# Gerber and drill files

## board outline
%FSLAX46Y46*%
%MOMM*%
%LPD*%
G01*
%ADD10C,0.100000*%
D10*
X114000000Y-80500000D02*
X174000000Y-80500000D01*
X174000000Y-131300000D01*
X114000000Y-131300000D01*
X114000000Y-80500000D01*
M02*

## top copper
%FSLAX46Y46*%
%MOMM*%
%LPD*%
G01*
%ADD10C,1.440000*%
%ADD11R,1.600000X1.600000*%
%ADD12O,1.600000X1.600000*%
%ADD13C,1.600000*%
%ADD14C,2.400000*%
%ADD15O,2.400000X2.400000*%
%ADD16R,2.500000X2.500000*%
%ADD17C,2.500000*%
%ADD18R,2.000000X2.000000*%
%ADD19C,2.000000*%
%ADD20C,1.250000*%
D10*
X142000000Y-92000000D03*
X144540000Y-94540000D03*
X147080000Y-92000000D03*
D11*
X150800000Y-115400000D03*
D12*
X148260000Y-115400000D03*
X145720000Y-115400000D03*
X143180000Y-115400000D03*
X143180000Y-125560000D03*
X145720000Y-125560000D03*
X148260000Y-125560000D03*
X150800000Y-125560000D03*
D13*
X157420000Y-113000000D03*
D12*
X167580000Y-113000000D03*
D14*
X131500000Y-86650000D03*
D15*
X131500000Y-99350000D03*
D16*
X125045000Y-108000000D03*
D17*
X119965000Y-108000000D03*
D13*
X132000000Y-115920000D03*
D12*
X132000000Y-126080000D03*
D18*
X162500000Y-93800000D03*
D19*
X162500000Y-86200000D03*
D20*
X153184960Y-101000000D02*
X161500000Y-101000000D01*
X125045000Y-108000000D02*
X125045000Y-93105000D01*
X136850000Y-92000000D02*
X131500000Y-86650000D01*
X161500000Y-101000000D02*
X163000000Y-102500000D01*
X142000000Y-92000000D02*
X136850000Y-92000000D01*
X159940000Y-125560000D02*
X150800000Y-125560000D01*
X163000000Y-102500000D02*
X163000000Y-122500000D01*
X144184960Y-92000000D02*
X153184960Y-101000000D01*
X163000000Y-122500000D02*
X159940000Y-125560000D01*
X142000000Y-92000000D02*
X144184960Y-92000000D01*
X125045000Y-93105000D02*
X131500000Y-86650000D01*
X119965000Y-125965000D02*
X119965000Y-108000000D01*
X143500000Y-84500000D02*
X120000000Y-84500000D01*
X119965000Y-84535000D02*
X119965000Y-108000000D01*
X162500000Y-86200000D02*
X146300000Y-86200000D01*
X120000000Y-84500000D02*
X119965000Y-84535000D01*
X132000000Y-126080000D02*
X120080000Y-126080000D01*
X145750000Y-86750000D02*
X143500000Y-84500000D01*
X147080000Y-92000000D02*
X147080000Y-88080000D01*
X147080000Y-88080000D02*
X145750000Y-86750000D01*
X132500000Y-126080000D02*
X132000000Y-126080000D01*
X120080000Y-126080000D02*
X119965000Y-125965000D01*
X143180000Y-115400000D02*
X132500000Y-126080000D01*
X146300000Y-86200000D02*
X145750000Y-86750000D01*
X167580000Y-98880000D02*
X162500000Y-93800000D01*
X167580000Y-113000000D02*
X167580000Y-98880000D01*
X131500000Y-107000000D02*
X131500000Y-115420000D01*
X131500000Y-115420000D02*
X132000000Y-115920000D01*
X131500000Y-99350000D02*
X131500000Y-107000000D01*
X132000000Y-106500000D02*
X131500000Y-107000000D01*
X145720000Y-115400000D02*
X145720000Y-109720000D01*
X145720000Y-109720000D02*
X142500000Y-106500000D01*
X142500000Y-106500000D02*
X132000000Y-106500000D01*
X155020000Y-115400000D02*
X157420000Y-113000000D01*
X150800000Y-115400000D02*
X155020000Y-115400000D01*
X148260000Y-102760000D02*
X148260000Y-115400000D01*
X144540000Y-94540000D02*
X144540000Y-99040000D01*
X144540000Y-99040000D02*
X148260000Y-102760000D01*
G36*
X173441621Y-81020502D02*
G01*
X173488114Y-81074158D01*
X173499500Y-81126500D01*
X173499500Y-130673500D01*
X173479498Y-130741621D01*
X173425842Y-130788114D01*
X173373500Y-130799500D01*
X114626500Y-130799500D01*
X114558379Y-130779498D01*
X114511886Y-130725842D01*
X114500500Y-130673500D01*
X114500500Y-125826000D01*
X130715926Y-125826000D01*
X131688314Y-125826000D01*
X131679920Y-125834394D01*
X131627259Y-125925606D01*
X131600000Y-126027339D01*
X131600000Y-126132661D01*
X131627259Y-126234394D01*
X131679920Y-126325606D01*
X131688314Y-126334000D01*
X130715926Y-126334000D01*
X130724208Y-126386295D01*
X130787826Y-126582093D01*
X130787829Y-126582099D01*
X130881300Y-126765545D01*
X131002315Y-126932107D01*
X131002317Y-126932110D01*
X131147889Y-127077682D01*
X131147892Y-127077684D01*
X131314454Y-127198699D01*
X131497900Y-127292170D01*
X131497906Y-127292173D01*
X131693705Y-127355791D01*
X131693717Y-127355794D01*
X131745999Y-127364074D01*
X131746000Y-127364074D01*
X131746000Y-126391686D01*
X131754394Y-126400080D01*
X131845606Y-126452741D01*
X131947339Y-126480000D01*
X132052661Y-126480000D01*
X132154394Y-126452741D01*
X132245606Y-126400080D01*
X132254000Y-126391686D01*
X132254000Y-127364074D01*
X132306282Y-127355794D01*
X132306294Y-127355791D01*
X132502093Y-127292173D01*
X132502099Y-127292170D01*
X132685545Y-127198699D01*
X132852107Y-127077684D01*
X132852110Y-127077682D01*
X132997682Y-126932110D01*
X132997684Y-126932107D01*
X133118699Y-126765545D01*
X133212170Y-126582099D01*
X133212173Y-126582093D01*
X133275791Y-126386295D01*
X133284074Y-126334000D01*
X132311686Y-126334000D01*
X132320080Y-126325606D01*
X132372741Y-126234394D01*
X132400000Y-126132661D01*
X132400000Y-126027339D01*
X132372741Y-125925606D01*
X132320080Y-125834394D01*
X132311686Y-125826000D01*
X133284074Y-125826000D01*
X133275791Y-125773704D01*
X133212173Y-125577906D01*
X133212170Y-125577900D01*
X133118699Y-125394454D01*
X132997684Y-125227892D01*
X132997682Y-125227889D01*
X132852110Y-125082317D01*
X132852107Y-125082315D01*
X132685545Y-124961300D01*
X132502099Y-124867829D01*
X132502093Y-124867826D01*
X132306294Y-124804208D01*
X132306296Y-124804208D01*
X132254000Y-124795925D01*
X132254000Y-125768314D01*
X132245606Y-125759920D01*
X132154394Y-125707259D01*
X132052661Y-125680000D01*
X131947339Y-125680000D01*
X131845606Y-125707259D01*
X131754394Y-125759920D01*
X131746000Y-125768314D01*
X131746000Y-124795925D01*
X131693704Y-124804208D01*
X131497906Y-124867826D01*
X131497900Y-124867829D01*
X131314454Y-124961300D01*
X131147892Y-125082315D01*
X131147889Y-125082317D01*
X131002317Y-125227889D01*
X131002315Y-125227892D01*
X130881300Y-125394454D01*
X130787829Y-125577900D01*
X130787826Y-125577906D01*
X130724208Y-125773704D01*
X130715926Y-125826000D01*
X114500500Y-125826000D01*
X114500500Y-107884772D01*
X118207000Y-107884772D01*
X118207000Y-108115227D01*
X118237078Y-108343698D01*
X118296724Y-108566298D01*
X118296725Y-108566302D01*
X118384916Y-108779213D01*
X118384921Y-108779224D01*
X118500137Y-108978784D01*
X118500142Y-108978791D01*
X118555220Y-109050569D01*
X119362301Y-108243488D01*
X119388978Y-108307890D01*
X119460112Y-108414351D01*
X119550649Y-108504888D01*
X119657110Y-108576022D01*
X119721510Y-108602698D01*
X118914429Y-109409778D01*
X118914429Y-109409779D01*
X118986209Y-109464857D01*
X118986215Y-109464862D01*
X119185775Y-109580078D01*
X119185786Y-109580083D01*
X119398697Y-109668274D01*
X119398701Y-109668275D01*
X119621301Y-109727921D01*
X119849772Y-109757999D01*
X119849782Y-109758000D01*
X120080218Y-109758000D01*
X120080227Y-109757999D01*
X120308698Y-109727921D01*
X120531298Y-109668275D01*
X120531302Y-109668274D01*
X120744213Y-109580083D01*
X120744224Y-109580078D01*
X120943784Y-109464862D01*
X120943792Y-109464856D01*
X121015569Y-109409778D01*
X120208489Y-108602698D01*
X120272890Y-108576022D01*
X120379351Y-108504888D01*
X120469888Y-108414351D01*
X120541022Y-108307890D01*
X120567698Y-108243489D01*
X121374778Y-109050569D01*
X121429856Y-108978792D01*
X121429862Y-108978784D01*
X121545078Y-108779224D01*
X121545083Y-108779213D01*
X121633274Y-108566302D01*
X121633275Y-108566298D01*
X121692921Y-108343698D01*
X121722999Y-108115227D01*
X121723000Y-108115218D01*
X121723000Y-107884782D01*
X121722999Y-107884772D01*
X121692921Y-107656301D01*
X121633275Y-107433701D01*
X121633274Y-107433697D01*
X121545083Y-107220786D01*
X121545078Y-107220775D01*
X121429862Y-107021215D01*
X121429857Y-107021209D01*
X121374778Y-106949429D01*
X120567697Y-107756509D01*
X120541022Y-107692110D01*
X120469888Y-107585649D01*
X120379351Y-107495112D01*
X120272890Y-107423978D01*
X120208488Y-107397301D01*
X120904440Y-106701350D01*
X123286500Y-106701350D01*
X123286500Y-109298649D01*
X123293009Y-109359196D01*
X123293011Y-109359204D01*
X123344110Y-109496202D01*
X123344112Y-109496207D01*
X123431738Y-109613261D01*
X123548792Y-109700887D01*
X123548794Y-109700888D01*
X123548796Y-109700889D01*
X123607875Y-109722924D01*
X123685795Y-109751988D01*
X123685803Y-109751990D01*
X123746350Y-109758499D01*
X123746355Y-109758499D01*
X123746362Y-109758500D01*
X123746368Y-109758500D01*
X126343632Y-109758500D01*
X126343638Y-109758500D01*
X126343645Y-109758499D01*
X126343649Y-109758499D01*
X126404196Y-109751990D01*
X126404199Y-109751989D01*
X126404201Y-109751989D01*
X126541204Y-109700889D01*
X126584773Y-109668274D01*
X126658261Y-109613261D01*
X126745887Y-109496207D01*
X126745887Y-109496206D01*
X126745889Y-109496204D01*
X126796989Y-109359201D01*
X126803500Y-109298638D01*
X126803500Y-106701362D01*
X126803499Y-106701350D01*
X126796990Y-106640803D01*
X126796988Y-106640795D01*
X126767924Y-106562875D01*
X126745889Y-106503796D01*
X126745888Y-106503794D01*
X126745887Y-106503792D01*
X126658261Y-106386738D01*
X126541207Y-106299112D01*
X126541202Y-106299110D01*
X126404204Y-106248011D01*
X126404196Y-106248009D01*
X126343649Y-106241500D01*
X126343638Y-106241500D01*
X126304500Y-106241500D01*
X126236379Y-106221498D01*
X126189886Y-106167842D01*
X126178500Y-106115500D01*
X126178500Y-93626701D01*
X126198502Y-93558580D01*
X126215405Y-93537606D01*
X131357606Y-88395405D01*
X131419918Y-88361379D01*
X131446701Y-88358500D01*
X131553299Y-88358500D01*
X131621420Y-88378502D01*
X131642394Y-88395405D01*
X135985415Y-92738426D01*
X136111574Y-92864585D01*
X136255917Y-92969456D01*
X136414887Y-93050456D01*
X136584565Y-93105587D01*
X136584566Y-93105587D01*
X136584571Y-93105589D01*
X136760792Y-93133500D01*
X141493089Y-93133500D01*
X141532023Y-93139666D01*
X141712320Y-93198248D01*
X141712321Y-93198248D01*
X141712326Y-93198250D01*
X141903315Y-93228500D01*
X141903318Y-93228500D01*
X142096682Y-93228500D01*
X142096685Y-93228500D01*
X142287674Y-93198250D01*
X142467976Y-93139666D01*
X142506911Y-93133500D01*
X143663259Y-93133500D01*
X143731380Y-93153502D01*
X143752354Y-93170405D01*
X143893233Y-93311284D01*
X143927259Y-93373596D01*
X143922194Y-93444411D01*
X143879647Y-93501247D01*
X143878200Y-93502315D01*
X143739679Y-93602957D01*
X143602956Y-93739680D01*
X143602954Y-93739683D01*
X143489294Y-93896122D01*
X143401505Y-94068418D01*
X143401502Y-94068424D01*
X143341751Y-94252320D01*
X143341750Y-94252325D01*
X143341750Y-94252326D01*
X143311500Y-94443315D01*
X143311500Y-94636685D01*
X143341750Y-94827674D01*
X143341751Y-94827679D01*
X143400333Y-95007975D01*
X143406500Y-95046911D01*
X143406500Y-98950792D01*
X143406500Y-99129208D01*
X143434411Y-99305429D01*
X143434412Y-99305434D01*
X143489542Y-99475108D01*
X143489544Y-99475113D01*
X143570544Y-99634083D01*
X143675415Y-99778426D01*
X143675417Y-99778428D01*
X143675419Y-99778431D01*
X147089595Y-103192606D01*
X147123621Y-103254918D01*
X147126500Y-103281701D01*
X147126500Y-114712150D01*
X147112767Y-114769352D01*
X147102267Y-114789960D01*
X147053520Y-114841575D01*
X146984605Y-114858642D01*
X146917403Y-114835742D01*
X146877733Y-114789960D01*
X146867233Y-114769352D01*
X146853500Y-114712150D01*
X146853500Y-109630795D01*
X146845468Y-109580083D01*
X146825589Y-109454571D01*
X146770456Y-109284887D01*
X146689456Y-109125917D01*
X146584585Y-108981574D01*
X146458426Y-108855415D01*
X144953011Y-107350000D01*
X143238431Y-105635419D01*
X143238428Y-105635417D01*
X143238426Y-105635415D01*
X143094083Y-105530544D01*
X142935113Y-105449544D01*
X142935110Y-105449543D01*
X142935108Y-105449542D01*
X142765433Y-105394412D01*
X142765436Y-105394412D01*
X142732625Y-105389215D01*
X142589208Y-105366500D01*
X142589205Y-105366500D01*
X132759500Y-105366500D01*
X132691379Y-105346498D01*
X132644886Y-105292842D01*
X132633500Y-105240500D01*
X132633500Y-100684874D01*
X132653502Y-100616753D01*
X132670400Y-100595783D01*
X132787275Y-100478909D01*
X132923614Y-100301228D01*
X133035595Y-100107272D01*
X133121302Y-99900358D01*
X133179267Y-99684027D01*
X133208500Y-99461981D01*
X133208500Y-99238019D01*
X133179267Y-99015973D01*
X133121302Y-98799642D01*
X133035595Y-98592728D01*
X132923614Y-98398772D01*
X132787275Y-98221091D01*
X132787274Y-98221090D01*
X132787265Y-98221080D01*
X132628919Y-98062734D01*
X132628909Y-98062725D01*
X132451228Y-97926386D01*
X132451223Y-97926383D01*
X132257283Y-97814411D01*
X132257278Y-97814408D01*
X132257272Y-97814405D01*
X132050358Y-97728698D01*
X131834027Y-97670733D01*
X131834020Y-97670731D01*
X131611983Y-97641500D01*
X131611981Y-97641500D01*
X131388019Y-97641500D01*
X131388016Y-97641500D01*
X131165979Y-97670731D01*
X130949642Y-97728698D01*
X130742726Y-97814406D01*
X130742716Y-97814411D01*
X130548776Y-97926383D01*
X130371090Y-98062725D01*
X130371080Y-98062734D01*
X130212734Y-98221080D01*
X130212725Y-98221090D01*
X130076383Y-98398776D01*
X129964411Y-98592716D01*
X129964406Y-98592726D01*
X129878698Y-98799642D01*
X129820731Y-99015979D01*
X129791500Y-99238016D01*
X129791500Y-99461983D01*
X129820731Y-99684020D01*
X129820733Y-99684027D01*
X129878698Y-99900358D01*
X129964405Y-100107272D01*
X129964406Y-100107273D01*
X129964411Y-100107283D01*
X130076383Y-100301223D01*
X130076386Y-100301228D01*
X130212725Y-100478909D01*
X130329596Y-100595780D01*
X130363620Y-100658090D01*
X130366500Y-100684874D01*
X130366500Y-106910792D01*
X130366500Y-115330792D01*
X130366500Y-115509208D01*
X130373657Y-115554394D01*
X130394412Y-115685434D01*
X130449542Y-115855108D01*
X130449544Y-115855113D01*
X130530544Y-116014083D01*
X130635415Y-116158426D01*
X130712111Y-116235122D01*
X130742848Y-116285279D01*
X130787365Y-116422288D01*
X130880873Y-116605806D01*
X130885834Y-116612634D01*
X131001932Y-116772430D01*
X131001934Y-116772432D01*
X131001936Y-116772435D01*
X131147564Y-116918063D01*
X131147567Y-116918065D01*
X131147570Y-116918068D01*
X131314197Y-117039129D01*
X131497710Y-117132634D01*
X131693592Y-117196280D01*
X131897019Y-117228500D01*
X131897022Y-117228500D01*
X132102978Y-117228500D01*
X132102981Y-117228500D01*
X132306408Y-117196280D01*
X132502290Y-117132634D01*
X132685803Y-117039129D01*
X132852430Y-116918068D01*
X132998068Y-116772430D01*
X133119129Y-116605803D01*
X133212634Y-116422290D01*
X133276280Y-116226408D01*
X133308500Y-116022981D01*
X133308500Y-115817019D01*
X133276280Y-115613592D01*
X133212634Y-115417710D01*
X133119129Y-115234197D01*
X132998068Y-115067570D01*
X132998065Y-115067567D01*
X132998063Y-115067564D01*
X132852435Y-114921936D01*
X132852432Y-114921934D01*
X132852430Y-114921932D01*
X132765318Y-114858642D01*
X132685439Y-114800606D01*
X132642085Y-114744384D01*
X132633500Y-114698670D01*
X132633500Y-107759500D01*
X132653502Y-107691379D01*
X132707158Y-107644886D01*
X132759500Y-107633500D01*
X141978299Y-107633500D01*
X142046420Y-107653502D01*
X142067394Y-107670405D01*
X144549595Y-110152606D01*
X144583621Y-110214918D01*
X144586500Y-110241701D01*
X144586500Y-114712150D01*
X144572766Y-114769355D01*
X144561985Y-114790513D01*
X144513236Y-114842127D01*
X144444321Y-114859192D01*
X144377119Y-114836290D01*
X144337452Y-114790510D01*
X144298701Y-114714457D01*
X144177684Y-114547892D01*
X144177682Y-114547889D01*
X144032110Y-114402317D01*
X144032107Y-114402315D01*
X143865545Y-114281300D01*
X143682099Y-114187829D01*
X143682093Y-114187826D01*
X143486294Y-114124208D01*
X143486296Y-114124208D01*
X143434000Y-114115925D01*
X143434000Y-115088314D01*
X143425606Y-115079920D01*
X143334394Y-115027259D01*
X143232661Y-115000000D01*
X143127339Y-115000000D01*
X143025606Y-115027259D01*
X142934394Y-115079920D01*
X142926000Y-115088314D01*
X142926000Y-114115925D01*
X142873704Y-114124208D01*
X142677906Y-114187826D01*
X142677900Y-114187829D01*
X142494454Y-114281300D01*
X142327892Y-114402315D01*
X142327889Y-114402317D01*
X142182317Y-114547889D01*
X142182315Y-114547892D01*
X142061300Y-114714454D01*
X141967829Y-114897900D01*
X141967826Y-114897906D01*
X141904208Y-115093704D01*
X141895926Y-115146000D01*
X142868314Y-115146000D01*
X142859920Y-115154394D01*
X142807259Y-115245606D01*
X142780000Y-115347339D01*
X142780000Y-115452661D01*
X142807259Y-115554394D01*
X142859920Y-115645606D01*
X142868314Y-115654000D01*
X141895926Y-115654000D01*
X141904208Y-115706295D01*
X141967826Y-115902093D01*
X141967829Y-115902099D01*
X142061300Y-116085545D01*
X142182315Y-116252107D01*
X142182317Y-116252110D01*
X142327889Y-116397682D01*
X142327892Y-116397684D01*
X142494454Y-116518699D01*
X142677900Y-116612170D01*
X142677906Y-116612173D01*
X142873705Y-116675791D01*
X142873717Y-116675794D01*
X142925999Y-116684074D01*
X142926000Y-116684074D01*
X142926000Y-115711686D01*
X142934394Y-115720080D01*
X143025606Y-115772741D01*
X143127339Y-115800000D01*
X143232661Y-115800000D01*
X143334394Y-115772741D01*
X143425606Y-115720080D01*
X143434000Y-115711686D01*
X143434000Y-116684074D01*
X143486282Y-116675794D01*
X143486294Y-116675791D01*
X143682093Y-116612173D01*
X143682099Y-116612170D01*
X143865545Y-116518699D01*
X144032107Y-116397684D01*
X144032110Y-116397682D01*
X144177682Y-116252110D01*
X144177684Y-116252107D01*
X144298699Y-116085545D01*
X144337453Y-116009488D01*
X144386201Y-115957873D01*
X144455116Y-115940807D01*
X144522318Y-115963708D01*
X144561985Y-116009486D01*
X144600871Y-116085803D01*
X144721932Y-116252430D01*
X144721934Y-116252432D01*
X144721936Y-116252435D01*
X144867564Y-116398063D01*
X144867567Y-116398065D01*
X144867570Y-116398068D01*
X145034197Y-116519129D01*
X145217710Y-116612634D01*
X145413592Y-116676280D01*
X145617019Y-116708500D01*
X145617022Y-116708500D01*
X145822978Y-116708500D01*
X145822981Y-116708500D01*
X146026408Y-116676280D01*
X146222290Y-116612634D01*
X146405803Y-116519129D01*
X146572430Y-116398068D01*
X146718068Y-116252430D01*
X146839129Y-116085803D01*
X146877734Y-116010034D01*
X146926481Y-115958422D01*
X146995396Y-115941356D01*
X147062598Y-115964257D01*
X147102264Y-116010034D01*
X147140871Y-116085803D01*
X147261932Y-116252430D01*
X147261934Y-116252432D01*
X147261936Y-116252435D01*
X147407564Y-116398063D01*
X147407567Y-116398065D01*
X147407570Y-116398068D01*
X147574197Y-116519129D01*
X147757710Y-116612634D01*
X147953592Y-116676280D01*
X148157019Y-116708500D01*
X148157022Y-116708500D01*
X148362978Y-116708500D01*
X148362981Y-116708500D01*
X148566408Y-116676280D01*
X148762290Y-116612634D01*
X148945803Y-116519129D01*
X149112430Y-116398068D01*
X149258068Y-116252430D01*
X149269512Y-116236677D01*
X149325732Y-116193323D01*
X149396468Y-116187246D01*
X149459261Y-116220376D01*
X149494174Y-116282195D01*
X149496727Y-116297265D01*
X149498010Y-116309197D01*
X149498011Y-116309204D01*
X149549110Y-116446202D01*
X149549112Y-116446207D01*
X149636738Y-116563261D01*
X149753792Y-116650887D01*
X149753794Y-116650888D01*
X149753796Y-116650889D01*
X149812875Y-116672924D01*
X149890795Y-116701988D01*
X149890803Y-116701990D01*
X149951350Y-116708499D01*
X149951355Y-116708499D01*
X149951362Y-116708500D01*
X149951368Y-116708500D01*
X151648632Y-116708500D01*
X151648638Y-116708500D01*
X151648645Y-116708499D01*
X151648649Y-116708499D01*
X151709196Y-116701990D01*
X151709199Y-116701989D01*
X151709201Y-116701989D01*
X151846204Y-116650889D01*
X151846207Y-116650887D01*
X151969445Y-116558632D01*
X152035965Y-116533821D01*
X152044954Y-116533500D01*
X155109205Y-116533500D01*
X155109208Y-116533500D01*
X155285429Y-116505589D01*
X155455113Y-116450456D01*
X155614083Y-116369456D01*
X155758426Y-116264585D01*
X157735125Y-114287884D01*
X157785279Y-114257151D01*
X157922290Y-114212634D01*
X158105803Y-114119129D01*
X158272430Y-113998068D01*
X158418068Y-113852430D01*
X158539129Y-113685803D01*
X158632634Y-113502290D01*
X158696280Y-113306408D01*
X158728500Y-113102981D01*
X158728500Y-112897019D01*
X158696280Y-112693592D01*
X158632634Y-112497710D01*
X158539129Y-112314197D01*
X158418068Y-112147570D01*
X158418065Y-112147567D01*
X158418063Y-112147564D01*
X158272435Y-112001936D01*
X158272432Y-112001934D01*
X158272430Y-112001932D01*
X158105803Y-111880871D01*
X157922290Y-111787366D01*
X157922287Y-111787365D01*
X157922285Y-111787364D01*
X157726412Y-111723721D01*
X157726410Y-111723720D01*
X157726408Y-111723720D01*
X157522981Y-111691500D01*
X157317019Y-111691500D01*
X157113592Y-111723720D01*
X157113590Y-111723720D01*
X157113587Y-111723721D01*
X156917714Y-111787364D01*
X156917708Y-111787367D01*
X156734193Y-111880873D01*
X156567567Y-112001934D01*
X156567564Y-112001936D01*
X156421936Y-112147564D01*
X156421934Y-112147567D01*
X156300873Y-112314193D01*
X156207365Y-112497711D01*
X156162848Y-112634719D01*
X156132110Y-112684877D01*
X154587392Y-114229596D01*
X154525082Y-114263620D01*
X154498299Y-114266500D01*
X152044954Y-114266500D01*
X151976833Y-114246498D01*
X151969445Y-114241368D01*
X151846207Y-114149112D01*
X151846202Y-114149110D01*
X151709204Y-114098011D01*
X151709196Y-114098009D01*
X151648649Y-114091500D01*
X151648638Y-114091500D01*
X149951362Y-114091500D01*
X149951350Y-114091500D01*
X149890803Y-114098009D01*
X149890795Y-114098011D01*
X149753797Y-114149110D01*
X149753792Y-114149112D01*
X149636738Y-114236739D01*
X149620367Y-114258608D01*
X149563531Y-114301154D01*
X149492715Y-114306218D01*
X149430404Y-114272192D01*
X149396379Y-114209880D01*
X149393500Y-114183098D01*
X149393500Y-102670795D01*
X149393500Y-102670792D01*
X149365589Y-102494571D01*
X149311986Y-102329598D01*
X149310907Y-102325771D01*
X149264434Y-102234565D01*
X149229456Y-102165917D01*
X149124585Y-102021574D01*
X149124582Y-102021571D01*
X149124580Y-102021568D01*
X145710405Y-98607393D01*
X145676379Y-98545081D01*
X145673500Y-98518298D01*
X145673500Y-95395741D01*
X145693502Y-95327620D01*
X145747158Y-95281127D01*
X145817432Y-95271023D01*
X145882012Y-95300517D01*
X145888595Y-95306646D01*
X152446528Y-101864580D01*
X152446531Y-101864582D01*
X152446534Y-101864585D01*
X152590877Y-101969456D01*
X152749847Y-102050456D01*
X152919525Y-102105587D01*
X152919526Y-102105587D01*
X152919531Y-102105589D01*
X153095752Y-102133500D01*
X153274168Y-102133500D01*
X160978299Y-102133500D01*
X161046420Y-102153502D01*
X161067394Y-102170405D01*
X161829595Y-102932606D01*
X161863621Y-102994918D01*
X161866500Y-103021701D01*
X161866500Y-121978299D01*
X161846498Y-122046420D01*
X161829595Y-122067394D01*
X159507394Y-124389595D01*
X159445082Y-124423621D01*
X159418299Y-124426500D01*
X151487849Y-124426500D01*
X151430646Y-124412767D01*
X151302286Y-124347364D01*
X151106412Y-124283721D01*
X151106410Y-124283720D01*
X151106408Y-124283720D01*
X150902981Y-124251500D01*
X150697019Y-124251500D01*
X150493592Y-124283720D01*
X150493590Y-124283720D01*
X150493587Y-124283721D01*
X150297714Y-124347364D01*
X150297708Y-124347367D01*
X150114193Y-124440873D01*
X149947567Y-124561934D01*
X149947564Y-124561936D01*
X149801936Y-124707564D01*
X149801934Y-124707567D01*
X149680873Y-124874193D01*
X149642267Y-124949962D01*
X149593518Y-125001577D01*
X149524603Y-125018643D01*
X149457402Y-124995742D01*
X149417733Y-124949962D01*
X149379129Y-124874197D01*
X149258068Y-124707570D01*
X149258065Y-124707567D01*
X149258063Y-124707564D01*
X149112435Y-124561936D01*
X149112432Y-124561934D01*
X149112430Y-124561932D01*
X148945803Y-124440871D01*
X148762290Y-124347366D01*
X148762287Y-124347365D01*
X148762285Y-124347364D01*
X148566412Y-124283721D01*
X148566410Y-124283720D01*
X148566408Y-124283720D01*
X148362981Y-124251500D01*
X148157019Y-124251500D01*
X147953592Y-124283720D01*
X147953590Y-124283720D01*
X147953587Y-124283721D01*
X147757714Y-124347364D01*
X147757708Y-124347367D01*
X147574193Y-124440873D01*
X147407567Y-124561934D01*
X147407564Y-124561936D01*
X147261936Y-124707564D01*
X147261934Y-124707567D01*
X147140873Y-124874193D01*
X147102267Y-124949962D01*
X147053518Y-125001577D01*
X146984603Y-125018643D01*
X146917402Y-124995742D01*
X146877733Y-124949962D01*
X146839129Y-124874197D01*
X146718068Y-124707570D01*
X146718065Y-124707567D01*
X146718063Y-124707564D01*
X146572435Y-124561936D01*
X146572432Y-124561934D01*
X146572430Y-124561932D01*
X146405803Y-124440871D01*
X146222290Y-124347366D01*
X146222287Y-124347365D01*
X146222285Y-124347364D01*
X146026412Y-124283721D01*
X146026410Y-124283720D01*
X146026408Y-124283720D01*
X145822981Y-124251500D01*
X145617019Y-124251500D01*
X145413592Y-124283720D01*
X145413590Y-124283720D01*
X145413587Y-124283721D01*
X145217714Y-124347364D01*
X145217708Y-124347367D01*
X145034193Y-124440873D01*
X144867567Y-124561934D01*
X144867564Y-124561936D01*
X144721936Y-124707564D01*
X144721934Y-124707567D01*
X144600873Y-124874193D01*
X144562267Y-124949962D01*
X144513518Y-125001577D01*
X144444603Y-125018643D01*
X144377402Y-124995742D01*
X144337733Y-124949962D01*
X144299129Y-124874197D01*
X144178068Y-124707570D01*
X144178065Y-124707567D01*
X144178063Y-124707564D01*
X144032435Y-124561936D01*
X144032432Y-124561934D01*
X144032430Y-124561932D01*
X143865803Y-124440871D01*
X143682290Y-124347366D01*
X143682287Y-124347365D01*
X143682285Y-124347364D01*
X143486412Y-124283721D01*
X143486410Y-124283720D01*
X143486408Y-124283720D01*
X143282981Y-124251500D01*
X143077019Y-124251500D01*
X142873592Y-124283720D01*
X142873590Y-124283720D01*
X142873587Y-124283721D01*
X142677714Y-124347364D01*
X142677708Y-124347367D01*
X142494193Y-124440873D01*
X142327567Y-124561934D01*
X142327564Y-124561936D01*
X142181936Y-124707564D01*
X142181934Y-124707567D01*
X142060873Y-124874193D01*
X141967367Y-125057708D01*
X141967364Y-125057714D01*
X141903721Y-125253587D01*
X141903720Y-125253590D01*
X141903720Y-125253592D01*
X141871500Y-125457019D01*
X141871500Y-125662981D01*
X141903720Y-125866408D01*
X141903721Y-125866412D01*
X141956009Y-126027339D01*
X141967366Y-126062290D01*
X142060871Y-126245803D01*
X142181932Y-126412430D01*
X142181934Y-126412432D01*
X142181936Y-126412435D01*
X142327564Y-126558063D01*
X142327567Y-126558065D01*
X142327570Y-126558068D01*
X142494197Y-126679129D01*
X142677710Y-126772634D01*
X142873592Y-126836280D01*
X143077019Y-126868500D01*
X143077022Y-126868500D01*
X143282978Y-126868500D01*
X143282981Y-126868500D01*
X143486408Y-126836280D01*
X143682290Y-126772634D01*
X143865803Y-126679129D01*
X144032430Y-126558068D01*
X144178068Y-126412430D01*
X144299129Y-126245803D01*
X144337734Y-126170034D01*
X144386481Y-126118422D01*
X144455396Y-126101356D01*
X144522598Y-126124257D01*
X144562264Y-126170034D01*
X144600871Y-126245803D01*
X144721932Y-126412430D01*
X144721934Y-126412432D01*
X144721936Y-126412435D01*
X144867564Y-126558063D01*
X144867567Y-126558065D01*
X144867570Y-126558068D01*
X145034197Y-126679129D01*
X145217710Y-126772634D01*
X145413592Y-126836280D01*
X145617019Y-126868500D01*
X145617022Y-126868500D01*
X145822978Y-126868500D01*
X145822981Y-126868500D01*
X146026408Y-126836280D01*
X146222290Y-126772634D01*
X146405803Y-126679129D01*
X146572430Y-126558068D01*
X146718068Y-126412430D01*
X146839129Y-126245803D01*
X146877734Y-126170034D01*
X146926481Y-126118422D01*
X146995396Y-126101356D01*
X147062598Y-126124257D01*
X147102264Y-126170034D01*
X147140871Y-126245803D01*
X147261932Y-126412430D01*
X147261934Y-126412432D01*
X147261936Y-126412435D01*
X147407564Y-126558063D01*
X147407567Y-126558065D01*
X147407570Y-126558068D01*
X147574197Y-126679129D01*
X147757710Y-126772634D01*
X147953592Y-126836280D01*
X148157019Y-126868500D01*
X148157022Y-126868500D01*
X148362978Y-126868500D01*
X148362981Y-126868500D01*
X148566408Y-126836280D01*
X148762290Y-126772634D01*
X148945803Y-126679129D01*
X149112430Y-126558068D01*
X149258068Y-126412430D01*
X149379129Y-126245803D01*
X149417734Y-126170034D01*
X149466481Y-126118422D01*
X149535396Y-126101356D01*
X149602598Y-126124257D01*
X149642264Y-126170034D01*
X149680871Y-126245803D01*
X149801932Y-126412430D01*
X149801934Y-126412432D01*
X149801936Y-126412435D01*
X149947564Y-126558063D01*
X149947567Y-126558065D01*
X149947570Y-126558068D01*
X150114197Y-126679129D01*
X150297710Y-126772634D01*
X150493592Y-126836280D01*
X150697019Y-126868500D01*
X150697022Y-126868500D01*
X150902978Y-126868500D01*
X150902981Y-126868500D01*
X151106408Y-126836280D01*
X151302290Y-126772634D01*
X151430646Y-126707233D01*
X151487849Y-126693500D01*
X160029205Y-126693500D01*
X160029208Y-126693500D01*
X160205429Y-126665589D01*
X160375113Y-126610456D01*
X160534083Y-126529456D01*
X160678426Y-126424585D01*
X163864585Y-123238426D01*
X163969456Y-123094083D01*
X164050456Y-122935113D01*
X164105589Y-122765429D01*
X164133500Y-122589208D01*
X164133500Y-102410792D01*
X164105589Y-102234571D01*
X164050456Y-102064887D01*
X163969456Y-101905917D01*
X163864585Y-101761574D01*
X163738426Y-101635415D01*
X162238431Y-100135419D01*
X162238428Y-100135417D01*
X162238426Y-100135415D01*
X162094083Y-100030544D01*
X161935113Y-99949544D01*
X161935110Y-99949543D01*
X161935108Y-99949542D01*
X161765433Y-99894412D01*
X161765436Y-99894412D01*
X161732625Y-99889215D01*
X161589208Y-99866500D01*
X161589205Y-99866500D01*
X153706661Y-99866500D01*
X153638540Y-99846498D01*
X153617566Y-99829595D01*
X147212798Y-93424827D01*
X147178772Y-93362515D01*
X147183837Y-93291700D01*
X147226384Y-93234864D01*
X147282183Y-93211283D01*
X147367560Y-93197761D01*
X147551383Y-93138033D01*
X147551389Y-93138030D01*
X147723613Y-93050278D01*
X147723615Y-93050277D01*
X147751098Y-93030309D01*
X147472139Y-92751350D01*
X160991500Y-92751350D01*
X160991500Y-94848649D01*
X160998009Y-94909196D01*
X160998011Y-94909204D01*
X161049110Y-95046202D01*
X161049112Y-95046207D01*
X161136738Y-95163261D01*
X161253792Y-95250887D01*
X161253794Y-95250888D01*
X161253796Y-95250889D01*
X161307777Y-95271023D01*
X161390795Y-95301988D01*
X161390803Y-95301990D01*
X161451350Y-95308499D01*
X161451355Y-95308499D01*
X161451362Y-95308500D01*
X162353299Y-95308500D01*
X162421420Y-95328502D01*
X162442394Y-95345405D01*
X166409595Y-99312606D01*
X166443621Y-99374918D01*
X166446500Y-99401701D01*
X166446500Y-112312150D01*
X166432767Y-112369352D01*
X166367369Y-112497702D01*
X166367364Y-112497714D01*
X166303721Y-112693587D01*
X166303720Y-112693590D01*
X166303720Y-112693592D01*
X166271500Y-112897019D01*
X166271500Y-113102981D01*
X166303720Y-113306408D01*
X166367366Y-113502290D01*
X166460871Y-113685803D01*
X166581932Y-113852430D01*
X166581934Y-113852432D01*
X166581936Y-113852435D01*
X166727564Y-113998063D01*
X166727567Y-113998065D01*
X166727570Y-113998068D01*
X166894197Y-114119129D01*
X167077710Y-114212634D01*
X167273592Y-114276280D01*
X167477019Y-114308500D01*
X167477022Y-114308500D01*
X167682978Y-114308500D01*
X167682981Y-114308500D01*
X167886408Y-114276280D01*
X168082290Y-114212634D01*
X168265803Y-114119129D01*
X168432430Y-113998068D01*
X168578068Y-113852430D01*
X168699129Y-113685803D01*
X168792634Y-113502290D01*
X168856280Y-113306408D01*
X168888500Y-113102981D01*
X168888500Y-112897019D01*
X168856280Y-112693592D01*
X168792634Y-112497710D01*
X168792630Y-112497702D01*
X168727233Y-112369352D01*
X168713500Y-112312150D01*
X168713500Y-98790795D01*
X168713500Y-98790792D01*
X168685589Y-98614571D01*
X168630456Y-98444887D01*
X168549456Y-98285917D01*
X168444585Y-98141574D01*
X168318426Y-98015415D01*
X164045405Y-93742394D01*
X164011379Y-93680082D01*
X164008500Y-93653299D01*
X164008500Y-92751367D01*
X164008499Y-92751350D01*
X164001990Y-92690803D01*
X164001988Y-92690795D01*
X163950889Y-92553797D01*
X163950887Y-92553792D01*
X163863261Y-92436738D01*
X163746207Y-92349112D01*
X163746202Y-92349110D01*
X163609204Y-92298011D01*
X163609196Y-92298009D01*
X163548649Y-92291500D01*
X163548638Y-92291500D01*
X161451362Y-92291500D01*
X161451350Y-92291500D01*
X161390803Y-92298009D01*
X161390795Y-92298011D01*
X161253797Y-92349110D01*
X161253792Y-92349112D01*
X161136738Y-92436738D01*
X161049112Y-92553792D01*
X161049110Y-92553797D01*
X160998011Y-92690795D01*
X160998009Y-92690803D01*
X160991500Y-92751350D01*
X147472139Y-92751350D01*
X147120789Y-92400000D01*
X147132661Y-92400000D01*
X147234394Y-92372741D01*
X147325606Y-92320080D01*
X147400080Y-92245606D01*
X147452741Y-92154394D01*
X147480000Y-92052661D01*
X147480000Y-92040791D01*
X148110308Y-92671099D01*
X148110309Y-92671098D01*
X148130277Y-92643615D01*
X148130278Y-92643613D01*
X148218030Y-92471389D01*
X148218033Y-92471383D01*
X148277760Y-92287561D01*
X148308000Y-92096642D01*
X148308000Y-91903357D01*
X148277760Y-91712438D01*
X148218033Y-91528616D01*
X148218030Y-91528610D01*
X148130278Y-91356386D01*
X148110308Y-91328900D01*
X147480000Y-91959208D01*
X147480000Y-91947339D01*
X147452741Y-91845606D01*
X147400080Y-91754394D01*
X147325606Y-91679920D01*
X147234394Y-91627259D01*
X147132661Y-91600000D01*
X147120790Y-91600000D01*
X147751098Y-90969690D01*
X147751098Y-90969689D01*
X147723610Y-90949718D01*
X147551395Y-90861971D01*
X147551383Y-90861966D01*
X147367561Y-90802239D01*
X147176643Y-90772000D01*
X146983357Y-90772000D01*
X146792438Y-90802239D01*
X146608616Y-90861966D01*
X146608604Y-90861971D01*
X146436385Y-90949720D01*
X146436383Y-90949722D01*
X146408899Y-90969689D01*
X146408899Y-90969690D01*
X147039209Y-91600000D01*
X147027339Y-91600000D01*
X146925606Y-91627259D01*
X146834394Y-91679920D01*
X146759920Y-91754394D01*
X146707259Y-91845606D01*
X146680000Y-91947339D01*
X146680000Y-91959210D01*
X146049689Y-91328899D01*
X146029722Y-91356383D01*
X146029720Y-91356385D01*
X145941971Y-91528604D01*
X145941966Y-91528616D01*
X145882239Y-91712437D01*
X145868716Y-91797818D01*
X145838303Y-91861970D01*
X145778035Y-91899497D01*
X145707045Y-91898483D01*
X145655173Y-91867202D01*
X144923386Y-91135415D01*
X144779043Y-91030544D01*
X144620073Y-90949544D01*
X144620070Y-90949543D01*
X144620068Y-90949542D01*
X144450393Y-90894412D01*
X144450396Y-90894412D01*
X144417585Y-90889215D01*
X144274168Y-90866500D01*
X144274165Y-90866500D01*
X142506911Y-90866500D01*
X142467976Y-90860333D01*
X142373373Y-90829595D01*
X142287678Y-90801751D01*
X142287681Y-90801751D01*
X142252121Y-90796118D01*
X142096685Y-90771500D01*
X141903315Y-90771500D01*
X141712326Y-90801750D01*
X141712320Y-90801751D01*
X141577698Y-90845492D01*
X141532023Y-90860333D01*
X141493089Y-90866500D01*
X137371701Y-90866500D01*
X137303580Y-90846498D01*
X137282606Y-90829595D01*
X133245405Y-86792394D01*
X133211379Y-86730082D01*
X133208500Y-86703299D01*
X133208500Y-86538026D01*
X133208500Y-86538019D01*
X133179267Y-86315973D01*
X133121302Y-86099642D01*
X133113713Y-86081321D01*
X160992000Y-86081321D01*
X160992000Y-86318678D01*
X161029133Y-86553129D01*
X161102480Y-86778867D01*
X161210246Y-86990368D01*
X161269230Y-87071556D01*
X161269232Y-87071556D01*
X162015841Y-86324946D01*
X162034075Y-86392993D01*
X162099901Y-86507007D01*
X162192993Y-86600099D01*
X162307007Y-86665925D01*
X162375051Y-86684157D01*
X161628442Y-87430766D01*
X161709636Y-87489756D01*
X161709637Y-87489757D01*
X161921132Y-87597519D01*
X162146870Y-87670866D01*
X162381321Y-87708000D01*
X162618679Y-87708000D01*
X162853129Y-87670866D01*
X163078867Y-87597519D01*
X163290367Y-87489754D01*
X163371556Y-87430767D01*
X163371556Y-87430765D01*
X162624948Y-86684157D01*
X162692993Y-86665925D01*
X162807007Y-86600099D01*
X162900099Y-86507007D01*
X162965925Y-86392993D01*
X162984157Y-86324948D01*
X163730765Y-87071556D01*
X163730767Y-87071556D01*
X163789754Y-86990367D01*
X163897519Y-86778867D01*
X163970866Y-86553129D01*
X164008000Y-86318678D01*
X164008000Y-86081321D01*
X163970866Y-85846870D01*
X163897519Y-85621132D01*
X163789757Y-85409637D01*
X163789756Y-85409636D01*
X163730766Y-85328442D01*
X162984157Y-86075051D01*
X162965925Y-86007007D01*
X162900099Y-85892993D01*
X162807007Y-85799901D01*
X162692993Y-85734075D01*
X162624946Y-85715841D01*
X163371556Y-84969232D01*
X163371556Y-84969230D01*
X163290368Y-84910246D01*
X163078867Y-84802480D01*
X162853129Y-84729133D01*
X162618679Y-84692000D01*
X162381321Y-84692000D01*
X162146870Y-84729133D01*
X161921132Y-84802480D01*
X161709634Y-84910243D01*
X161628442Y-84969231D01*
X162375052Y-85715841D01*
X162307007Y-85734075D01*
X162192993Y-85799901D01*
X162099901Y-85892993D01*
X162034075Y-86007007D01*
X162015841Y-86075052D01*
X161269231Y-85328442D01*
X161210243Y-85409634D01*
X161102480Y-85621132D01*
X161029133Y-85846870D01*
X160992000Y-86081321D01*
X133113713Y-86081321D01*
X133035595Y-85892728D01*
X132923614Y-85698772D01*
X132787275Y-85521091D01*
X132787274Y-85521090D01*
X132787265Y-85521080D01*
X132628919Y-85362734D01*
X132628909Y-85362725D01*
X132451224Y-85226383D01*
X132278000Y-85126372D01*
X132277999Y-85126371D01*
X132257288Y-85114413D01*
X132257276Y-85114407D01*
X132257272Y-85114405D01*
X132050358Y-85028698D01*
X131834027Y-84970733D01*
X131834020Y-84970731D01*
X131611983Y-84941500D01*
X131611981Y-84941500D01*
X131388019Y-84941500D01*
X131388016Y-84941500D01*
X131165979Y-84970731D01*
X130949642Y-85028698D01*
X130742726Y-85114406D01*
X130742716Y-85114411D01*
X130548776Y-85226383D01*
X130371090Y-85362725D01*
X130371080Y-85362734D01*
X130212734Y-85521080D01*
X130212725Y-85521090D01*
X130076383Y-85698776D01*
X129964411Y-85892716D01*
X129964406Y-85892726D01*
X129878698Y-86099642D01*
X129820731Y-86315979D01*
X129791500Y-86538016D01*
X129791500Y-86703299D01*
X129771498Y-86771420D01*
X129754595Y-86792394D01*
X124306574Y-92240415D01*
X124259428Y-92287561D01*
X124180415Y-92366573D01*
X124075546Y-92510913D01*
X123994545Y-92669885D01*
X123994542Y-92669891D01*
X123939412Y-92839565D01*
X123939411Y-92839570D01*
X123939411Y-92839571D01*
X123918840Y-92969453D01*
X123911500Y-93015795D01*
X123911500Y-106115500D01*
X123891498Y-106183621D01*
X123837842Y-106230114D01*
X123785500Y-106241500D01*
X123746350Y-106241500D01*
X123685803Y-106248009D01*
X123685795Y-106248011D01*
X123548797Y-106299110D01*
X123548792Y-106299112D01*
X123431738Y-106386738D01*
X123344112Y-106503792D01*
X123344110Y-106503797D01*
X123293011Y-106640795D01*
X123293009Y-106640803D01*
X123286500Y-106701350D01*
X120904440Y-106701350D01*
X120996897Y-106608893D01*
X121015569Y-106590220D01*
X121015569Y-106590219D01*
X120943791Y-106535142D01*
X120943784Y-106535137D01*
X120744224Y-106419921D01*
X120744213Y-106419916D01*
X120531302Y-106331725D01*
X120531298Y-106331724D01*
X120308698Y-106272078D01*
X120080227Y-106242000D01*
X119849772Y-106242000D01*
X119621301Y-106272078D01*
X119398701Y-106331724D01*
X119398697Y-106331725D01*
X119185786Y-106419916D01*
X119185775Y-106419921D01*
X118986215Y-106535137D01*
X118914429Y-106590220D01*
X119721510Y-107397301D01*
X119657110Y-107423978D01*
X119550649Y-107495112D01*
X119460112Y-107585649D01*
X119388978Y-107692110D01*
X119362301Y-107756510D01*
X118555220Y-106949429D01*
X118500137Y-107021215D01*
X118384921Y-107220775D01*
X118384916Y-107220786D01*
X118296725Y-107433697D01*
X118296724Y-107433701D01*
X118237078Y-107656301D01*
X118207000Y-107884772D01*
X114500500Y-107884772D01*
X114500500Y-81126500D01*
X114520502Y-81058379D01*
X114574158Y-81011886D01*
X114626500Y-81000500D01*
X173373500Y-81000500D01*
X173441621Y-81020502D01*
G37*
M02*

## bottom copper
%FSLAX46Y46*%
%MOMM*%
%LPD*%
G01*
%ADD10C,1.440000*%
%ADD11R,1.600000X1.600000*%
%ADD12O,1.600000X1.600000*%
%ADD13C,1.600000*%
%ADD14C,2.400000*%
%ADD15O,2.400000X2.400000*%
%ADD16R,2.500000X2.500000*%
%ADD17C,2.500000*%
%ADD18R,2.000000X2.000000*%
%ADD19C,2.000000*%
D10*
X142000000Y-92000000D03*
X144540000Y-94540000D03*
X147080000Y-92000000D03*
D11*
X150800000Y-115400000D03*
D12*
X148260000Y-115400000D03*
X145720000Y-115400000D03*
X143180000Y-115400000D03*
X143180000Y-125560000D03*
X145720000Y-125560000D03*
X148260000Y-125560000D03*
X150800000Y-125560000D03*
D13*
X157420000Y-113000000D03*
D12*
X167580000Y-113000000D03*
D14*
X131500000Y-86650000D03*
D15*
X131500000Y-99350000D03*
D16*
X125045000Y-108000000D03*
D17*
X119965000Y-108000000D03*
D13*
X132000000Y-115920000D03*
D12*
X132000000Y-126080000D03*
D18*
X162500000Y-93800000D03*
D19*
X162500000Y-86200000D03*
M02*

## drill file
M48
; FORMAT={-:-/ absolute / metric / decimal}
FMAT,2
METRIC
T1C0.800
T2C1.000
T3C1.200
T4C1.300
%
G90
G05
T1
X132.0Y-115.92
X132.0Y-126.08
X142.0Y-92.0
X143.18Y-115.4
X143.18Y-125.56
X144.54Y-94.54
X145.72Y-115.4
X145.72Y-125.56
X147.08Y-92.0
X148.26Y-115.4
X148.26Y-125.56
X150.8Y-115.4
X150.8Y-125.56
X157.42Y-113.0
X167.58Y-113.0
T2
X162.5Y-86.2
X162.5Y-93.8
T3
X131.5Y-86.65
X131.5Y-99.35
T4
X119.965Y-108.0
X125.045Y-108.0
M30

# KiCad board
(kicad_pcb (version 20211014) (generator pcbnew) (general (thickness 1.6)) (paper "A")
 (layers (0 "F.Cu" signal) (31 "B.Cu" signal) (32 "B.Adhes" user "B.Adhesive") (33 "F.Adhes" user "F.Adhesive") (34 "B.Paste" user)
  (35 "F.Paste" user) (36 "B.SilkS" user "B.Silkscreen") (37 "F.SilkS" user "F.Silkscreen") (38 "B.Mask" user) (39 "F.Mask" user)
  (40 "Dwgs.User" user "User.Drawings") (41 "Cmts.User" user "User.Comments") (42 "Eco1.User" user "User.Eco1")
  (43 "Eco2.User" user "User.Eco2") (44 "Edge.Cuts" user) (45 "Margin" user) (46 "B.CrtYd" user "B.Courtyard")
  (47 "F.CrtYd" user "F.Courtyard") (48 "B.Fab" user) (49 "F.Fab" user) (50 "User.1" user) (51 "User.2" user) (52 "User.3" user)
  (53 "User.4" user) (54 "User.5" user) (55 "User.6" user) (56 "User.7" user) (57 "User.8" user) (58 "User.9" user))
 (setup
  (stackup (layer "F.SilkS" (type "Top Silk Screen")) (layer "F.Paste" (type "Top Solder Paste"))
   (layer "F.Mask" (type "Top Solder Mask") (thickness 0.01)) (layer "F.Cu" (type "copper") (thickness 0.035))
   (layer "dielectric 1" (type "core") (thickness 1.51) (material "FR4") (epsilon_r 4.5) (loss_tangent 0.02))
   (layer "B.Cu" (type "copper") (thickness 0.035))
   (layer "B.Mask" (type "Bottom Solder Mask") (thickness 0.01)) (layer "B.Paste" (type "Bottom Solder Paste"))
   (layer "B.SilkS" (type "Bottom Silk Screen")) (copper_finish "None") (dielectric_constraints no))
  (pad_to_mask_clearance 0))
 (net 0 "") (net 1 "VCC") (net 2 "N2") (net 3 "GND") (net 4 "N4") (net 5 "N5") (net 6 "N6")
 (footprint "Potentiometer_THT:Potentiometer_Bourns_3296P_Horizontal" (layer "F.Cu") (at 142 92 90)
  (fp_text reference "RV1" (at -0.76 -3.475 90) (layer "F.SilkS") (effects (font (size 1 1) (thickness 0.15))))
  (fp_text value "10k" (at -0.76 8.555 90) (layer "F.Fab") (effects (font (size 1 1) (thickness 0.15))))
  (pad "1" thru_hole circle (at 0 0 90) (size 1.44 1.44) (drill 0.8) (layers *.Cu *.Mask) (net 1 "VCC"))
  (pad "2" thru_hole circle (at -2.54 2.54 90) (size 1.44 1.44) (drill 0.8) (layers *.Cu *.Mask) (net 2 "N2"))
  (pad "3" thru_hole circle (at 0 5.08 90) (size 1.44 1.44) (drill 0.8) (layers *.Cu *.Mask) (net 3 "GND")))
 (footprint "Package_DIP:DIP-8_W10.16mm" (layer "F.Cu") (at 150.8 115.4 -90)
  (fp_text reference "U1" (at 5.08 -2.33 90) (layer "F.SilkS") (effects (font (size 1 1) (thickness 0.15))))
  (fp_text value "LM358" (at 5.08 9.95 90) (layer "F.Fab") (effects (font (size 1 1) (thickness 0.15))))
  (pad "1" thru_hole rect (at 0 0 270) (size 1.6 1.6) (drill 0.8) (layers *.Cu *.Mask) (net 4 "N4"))
  (pad "2" thru_hole oval (at 0 2.54 270) (size 1.6 1.6) (drill 0.8) (layers *.Cu *.Mask) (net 2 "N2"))
  (pad "3" thru_hole oval (at 0 5.08 270) (size 1.6 1.6) (drill 0.8) (layers *.Cu *.Mask) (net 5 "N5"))
  (pad "4" thru_hole oval (at 0 7.62 270) (size 1.6 1.6) (drill 0.8) (layers *.Cu *.Mask) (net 3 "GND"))
  (pad "5" thru_hole oval (at 10.16 7.62 270) (size 1.6 1.6) (drill 0.8) (layers *.Cu *.Mask))
  (pad "6" thru_hole oval (at 10.16 5.08 270) (size 1.6 1.6) (drill 0.8) (layers *.Cu *.Mask))
  (pad "7" thru_hole oval (at 10.16 2.54 270) (size 1.6 1.6) (drill 0.8) (layers *.Cu *.Mask))
  (pad "8" thru_hole oval (at 10.16 0 270) (size 1.6 1.6) (drill 0.8) (layers *.Cu *.Mask) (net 1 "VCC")))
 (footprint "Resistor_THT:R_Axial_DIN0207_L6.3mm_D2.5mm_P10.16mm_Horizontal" (layer "F.Cu") (at 157.42 113)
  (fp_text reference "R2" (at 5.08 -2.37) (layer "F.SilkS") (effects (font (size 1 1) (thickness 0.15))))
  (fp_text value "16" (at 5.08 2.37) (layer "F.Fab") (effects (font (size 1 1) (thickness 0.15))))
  (pad "1" thru_hole circle (at 0 0) (size 1.6 1.6) (drill 0.8) (layers *.Cu *.Mask) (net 4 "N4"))
  (pad "2" thru_hole oval (at 10.16 0) (size 1.6 1.6) (drill 0.8) (layers *.Cu *.Mask) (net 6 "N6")))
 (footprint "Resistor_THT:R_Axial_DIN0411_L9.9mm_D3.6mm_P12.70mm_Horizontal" (layer "F.Cu") (at 131.5 86.65 -90)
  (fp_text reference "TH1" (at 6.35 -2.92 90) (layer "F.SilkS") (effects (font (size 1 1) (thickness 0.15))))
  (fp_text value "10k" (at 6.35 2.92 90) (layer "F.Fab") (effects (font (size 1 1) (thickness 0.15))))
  (pad "1" thru_hole circle (at 0 0 270) (size 2.4 2.4) (drill 1.2) (layers *.Cu *.Mask) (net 1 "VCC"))
  (pad "2" thru_hole oval (at 12.7 0 270) (size 2.4 2.4) (drill 1.2) (layers *.Cu *.Mask) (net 5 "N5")))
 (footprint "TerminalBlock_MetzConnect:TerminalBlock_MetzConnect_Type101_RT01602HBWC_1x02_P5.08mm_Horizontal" (layer "F.Cu")
  (at 125.045 108 180)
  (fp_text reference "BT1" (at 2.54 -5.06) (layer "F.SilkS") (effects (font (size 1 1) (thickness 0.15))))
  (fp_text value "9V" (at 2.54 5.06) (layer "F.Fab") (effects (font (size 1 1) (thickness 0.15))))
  (pad "1" thru_hole rect (at 0 0 180) (size 2.5 2.5) (drill 1.3) (layers *.Cu *.Mask) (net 1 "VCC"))
  (pad "2" thru_hole circle (at 5.08 0 180) (size 2.5 2.5) (drill 1.3) (layers *.Cu *.Mask) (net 3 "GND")))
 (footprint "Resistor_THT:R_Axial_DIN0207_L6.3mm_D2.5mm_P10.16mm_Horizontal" (layer "F.Cu") (at 132 115.92 -90)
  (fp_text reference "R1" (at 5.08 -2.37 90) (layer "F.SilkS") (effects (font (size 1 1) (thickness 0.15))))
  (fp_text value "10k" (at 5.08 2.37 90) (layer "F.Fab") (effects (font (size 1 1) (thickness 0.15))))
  (pad "1" thru_hole circle (at 0 0 270) (size 1.6 1.6) (drill 0.8) (layers *.Cu *.Mask) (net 5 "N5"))
  (pad "2" thru_hole oval (at 10.16 0 270) (size 1.6 1.6) (drill 0.8) (layers *.Cu *.Mask) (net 3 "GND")))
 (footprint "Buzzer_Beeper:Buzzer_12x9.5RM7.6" (layer "F.Cu") (at 162.5 93.8 90)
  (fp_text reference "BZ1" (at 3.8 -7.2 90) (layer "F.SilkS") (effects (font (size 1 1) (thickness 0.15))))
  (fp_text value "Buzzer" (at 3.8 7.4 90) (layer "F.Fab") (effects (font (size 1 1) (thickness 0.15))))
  (pad "1" thru_hole rect (at 0 0 90) (size 2 2) (drill 1) (layers *.Cu *.Mask) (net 6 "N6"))
  (pad "2" thru_hole circle (at 7.6 0 90) (size 2 2) (drill 1) (layers *.Cu *.Mask) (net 3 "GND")))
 (gr_rect (start 114 80.5) (end 174 131.3) (layer "Edge.Cuts") (width 0.1) (fill none))
 (segment (start 153.18496 101) (end 161.5 101) (width 1.25) (layer "F.Cu") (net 1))
 (segment (start 125.045 108) (end 125.045 93.105) (width 1.25) (layer "F.Cu") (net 1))
 (segment (start 136.85 92) (end 131.5 86.65) (width 1.25) (layer "F.Cu") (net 1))
 (segment (start 161.5 101) (end 163 102.5) (width 1.25) (layer "F.Cu") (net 1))
 (segment (start 142 92) (end 136.85 92) (width 1.25) (layer "F.Cu") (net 1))
 (segment (start 159.94 125.56) (end 150.8 125.56) (width 1.25) (layer "F.Cu") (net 1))
 (segment (start 163 102.5) (end 163 122.5) (width 1.25) (layer "F.Cu") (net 1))
 (segment (start 144.18496 92) (end 153.18496 101) (width 1.25) (layer "F.Cu") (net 1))
 (segment (start 163 122.5) (end 159.94 125.56) (width 1.25) (layer "F.Cu") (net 1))
 (segment (start 142 92) (end 144.18496 92) (width 1.25) (layer "F.Cu") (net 1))
 (segment (start 125.045 93.105) (end 131.5 86.65) (width 1.25) (layer "F.Cu") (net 1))
 (segment (start 119.965 125.965) (end 119.965 108) (width 1.25) (layer "F.Cu") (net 3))
 (segment (start 143.5 84.5) (end 120 84.5) (width 1.25) (layer "F.Cu") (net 3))
 (segment (start 119.965 84.535) (end 119.965 108) (width 1.25) (layer "F.Cu") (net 3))
 (segment (start 162.5 86.2) (end 146.3 86.2) (width 1.25) (layer "F.Cu") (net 3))
 (segment (start 120 84.5) (end 119.965 84.535) (width 1.25) (layer "F.Cu") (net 3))
 (segment (start 132 126.08) (end 120.08 126.08) (width 1.25) (layer "F.Cu") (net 3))
 (segment (start 145.75 86.75) (end 143.5 84.5) (width 1.25) (layer "F.Cu") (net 3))
 (segment (start 147.08 92) (end 147.08 88.08) (width 1.25) (layer "F.Cu") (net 3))
 (segment (start 147.08 88.08) (end 145.75 86.75) (width 1.25) (layer "F.Cu") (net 3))
 (segment (start 132.5 126.08) (end 132 126.08) (width 1.25) (layer "F.Cu") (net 3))
 (segment (start 120.08 126.08) (end 119.965 125.965) (width 1.25) (layer "F.Cu") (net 3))
 (segment (start 143.18 115.4) (end 132.5 126.08) (width 1.25) (layer "F.Cu") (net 3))
 (segment (start 146.3 86.2) (end 145.75 86.75) (width 1.25) (layer "F.Cu") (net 3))
 (segment (start 167.58 98.88) (end 162.5 93.8) (width 1.25) (layer "F.Cu") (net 6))
 (segment (start 167.58 113) (end 167.58 98.88) (width 1.25) (layer "F.Cu") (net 6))
 (segment (start 131.5 107) (end 131.5 115.42) (width 1.25) (layer "F.Cu") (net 5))
 (segment (start 131.5 115.42) (end 132 115.92) (width 1.25) (layer "F.Cu") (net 5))
 (segment (start 131.5 99.35) (end 131.5 107) (width 1.25) (layer "F.Cu") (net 5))
 (segment (start 132 106.5) (end 131.5 107) (width 1.25) (layer "F.Cu") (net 5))
 (segment (start 145.72 115.4) (end 145.72 109.72) (width 1.25) (layer "F.Cu") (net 5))
 (segment (start 145.72 109.72) (end 142.5 106.5) (width 1.25) (layer "F.Cu") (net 5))
 (segment (start 142.5 106.5) (end 132 106.5) (width 1.25) (layer "F.Cu") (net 5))
 (segment (start 155.02 115.4) (end 157.42 113) (width 1.25) (layer "F.Cu") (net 4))
 (segment (start 150.8 115.4) (end 155.02 115.4) (width 1.25) (layer "F.Cu") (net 4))
 (segment (start 148.26 102.76) (end 148.26 115.4) (width 1.25) (layer "F.Cu") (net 2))
 (segment (start 144.54 94.54) (end 144.54 99.04) (width 1.25) (layer "F.Cu") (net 2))
 (segment (start 144.54 99.04) (end 148.26 102.76) (width 1.25) (layer "F.Cu") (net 2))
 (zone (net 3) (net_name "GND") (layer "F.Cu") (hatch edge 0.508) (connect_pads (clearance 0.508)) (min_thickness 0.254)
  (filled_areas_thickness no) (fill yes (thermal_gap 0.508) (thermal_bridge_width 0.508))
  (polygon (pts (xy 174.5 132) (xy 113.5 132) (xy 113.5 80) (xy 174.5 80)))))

